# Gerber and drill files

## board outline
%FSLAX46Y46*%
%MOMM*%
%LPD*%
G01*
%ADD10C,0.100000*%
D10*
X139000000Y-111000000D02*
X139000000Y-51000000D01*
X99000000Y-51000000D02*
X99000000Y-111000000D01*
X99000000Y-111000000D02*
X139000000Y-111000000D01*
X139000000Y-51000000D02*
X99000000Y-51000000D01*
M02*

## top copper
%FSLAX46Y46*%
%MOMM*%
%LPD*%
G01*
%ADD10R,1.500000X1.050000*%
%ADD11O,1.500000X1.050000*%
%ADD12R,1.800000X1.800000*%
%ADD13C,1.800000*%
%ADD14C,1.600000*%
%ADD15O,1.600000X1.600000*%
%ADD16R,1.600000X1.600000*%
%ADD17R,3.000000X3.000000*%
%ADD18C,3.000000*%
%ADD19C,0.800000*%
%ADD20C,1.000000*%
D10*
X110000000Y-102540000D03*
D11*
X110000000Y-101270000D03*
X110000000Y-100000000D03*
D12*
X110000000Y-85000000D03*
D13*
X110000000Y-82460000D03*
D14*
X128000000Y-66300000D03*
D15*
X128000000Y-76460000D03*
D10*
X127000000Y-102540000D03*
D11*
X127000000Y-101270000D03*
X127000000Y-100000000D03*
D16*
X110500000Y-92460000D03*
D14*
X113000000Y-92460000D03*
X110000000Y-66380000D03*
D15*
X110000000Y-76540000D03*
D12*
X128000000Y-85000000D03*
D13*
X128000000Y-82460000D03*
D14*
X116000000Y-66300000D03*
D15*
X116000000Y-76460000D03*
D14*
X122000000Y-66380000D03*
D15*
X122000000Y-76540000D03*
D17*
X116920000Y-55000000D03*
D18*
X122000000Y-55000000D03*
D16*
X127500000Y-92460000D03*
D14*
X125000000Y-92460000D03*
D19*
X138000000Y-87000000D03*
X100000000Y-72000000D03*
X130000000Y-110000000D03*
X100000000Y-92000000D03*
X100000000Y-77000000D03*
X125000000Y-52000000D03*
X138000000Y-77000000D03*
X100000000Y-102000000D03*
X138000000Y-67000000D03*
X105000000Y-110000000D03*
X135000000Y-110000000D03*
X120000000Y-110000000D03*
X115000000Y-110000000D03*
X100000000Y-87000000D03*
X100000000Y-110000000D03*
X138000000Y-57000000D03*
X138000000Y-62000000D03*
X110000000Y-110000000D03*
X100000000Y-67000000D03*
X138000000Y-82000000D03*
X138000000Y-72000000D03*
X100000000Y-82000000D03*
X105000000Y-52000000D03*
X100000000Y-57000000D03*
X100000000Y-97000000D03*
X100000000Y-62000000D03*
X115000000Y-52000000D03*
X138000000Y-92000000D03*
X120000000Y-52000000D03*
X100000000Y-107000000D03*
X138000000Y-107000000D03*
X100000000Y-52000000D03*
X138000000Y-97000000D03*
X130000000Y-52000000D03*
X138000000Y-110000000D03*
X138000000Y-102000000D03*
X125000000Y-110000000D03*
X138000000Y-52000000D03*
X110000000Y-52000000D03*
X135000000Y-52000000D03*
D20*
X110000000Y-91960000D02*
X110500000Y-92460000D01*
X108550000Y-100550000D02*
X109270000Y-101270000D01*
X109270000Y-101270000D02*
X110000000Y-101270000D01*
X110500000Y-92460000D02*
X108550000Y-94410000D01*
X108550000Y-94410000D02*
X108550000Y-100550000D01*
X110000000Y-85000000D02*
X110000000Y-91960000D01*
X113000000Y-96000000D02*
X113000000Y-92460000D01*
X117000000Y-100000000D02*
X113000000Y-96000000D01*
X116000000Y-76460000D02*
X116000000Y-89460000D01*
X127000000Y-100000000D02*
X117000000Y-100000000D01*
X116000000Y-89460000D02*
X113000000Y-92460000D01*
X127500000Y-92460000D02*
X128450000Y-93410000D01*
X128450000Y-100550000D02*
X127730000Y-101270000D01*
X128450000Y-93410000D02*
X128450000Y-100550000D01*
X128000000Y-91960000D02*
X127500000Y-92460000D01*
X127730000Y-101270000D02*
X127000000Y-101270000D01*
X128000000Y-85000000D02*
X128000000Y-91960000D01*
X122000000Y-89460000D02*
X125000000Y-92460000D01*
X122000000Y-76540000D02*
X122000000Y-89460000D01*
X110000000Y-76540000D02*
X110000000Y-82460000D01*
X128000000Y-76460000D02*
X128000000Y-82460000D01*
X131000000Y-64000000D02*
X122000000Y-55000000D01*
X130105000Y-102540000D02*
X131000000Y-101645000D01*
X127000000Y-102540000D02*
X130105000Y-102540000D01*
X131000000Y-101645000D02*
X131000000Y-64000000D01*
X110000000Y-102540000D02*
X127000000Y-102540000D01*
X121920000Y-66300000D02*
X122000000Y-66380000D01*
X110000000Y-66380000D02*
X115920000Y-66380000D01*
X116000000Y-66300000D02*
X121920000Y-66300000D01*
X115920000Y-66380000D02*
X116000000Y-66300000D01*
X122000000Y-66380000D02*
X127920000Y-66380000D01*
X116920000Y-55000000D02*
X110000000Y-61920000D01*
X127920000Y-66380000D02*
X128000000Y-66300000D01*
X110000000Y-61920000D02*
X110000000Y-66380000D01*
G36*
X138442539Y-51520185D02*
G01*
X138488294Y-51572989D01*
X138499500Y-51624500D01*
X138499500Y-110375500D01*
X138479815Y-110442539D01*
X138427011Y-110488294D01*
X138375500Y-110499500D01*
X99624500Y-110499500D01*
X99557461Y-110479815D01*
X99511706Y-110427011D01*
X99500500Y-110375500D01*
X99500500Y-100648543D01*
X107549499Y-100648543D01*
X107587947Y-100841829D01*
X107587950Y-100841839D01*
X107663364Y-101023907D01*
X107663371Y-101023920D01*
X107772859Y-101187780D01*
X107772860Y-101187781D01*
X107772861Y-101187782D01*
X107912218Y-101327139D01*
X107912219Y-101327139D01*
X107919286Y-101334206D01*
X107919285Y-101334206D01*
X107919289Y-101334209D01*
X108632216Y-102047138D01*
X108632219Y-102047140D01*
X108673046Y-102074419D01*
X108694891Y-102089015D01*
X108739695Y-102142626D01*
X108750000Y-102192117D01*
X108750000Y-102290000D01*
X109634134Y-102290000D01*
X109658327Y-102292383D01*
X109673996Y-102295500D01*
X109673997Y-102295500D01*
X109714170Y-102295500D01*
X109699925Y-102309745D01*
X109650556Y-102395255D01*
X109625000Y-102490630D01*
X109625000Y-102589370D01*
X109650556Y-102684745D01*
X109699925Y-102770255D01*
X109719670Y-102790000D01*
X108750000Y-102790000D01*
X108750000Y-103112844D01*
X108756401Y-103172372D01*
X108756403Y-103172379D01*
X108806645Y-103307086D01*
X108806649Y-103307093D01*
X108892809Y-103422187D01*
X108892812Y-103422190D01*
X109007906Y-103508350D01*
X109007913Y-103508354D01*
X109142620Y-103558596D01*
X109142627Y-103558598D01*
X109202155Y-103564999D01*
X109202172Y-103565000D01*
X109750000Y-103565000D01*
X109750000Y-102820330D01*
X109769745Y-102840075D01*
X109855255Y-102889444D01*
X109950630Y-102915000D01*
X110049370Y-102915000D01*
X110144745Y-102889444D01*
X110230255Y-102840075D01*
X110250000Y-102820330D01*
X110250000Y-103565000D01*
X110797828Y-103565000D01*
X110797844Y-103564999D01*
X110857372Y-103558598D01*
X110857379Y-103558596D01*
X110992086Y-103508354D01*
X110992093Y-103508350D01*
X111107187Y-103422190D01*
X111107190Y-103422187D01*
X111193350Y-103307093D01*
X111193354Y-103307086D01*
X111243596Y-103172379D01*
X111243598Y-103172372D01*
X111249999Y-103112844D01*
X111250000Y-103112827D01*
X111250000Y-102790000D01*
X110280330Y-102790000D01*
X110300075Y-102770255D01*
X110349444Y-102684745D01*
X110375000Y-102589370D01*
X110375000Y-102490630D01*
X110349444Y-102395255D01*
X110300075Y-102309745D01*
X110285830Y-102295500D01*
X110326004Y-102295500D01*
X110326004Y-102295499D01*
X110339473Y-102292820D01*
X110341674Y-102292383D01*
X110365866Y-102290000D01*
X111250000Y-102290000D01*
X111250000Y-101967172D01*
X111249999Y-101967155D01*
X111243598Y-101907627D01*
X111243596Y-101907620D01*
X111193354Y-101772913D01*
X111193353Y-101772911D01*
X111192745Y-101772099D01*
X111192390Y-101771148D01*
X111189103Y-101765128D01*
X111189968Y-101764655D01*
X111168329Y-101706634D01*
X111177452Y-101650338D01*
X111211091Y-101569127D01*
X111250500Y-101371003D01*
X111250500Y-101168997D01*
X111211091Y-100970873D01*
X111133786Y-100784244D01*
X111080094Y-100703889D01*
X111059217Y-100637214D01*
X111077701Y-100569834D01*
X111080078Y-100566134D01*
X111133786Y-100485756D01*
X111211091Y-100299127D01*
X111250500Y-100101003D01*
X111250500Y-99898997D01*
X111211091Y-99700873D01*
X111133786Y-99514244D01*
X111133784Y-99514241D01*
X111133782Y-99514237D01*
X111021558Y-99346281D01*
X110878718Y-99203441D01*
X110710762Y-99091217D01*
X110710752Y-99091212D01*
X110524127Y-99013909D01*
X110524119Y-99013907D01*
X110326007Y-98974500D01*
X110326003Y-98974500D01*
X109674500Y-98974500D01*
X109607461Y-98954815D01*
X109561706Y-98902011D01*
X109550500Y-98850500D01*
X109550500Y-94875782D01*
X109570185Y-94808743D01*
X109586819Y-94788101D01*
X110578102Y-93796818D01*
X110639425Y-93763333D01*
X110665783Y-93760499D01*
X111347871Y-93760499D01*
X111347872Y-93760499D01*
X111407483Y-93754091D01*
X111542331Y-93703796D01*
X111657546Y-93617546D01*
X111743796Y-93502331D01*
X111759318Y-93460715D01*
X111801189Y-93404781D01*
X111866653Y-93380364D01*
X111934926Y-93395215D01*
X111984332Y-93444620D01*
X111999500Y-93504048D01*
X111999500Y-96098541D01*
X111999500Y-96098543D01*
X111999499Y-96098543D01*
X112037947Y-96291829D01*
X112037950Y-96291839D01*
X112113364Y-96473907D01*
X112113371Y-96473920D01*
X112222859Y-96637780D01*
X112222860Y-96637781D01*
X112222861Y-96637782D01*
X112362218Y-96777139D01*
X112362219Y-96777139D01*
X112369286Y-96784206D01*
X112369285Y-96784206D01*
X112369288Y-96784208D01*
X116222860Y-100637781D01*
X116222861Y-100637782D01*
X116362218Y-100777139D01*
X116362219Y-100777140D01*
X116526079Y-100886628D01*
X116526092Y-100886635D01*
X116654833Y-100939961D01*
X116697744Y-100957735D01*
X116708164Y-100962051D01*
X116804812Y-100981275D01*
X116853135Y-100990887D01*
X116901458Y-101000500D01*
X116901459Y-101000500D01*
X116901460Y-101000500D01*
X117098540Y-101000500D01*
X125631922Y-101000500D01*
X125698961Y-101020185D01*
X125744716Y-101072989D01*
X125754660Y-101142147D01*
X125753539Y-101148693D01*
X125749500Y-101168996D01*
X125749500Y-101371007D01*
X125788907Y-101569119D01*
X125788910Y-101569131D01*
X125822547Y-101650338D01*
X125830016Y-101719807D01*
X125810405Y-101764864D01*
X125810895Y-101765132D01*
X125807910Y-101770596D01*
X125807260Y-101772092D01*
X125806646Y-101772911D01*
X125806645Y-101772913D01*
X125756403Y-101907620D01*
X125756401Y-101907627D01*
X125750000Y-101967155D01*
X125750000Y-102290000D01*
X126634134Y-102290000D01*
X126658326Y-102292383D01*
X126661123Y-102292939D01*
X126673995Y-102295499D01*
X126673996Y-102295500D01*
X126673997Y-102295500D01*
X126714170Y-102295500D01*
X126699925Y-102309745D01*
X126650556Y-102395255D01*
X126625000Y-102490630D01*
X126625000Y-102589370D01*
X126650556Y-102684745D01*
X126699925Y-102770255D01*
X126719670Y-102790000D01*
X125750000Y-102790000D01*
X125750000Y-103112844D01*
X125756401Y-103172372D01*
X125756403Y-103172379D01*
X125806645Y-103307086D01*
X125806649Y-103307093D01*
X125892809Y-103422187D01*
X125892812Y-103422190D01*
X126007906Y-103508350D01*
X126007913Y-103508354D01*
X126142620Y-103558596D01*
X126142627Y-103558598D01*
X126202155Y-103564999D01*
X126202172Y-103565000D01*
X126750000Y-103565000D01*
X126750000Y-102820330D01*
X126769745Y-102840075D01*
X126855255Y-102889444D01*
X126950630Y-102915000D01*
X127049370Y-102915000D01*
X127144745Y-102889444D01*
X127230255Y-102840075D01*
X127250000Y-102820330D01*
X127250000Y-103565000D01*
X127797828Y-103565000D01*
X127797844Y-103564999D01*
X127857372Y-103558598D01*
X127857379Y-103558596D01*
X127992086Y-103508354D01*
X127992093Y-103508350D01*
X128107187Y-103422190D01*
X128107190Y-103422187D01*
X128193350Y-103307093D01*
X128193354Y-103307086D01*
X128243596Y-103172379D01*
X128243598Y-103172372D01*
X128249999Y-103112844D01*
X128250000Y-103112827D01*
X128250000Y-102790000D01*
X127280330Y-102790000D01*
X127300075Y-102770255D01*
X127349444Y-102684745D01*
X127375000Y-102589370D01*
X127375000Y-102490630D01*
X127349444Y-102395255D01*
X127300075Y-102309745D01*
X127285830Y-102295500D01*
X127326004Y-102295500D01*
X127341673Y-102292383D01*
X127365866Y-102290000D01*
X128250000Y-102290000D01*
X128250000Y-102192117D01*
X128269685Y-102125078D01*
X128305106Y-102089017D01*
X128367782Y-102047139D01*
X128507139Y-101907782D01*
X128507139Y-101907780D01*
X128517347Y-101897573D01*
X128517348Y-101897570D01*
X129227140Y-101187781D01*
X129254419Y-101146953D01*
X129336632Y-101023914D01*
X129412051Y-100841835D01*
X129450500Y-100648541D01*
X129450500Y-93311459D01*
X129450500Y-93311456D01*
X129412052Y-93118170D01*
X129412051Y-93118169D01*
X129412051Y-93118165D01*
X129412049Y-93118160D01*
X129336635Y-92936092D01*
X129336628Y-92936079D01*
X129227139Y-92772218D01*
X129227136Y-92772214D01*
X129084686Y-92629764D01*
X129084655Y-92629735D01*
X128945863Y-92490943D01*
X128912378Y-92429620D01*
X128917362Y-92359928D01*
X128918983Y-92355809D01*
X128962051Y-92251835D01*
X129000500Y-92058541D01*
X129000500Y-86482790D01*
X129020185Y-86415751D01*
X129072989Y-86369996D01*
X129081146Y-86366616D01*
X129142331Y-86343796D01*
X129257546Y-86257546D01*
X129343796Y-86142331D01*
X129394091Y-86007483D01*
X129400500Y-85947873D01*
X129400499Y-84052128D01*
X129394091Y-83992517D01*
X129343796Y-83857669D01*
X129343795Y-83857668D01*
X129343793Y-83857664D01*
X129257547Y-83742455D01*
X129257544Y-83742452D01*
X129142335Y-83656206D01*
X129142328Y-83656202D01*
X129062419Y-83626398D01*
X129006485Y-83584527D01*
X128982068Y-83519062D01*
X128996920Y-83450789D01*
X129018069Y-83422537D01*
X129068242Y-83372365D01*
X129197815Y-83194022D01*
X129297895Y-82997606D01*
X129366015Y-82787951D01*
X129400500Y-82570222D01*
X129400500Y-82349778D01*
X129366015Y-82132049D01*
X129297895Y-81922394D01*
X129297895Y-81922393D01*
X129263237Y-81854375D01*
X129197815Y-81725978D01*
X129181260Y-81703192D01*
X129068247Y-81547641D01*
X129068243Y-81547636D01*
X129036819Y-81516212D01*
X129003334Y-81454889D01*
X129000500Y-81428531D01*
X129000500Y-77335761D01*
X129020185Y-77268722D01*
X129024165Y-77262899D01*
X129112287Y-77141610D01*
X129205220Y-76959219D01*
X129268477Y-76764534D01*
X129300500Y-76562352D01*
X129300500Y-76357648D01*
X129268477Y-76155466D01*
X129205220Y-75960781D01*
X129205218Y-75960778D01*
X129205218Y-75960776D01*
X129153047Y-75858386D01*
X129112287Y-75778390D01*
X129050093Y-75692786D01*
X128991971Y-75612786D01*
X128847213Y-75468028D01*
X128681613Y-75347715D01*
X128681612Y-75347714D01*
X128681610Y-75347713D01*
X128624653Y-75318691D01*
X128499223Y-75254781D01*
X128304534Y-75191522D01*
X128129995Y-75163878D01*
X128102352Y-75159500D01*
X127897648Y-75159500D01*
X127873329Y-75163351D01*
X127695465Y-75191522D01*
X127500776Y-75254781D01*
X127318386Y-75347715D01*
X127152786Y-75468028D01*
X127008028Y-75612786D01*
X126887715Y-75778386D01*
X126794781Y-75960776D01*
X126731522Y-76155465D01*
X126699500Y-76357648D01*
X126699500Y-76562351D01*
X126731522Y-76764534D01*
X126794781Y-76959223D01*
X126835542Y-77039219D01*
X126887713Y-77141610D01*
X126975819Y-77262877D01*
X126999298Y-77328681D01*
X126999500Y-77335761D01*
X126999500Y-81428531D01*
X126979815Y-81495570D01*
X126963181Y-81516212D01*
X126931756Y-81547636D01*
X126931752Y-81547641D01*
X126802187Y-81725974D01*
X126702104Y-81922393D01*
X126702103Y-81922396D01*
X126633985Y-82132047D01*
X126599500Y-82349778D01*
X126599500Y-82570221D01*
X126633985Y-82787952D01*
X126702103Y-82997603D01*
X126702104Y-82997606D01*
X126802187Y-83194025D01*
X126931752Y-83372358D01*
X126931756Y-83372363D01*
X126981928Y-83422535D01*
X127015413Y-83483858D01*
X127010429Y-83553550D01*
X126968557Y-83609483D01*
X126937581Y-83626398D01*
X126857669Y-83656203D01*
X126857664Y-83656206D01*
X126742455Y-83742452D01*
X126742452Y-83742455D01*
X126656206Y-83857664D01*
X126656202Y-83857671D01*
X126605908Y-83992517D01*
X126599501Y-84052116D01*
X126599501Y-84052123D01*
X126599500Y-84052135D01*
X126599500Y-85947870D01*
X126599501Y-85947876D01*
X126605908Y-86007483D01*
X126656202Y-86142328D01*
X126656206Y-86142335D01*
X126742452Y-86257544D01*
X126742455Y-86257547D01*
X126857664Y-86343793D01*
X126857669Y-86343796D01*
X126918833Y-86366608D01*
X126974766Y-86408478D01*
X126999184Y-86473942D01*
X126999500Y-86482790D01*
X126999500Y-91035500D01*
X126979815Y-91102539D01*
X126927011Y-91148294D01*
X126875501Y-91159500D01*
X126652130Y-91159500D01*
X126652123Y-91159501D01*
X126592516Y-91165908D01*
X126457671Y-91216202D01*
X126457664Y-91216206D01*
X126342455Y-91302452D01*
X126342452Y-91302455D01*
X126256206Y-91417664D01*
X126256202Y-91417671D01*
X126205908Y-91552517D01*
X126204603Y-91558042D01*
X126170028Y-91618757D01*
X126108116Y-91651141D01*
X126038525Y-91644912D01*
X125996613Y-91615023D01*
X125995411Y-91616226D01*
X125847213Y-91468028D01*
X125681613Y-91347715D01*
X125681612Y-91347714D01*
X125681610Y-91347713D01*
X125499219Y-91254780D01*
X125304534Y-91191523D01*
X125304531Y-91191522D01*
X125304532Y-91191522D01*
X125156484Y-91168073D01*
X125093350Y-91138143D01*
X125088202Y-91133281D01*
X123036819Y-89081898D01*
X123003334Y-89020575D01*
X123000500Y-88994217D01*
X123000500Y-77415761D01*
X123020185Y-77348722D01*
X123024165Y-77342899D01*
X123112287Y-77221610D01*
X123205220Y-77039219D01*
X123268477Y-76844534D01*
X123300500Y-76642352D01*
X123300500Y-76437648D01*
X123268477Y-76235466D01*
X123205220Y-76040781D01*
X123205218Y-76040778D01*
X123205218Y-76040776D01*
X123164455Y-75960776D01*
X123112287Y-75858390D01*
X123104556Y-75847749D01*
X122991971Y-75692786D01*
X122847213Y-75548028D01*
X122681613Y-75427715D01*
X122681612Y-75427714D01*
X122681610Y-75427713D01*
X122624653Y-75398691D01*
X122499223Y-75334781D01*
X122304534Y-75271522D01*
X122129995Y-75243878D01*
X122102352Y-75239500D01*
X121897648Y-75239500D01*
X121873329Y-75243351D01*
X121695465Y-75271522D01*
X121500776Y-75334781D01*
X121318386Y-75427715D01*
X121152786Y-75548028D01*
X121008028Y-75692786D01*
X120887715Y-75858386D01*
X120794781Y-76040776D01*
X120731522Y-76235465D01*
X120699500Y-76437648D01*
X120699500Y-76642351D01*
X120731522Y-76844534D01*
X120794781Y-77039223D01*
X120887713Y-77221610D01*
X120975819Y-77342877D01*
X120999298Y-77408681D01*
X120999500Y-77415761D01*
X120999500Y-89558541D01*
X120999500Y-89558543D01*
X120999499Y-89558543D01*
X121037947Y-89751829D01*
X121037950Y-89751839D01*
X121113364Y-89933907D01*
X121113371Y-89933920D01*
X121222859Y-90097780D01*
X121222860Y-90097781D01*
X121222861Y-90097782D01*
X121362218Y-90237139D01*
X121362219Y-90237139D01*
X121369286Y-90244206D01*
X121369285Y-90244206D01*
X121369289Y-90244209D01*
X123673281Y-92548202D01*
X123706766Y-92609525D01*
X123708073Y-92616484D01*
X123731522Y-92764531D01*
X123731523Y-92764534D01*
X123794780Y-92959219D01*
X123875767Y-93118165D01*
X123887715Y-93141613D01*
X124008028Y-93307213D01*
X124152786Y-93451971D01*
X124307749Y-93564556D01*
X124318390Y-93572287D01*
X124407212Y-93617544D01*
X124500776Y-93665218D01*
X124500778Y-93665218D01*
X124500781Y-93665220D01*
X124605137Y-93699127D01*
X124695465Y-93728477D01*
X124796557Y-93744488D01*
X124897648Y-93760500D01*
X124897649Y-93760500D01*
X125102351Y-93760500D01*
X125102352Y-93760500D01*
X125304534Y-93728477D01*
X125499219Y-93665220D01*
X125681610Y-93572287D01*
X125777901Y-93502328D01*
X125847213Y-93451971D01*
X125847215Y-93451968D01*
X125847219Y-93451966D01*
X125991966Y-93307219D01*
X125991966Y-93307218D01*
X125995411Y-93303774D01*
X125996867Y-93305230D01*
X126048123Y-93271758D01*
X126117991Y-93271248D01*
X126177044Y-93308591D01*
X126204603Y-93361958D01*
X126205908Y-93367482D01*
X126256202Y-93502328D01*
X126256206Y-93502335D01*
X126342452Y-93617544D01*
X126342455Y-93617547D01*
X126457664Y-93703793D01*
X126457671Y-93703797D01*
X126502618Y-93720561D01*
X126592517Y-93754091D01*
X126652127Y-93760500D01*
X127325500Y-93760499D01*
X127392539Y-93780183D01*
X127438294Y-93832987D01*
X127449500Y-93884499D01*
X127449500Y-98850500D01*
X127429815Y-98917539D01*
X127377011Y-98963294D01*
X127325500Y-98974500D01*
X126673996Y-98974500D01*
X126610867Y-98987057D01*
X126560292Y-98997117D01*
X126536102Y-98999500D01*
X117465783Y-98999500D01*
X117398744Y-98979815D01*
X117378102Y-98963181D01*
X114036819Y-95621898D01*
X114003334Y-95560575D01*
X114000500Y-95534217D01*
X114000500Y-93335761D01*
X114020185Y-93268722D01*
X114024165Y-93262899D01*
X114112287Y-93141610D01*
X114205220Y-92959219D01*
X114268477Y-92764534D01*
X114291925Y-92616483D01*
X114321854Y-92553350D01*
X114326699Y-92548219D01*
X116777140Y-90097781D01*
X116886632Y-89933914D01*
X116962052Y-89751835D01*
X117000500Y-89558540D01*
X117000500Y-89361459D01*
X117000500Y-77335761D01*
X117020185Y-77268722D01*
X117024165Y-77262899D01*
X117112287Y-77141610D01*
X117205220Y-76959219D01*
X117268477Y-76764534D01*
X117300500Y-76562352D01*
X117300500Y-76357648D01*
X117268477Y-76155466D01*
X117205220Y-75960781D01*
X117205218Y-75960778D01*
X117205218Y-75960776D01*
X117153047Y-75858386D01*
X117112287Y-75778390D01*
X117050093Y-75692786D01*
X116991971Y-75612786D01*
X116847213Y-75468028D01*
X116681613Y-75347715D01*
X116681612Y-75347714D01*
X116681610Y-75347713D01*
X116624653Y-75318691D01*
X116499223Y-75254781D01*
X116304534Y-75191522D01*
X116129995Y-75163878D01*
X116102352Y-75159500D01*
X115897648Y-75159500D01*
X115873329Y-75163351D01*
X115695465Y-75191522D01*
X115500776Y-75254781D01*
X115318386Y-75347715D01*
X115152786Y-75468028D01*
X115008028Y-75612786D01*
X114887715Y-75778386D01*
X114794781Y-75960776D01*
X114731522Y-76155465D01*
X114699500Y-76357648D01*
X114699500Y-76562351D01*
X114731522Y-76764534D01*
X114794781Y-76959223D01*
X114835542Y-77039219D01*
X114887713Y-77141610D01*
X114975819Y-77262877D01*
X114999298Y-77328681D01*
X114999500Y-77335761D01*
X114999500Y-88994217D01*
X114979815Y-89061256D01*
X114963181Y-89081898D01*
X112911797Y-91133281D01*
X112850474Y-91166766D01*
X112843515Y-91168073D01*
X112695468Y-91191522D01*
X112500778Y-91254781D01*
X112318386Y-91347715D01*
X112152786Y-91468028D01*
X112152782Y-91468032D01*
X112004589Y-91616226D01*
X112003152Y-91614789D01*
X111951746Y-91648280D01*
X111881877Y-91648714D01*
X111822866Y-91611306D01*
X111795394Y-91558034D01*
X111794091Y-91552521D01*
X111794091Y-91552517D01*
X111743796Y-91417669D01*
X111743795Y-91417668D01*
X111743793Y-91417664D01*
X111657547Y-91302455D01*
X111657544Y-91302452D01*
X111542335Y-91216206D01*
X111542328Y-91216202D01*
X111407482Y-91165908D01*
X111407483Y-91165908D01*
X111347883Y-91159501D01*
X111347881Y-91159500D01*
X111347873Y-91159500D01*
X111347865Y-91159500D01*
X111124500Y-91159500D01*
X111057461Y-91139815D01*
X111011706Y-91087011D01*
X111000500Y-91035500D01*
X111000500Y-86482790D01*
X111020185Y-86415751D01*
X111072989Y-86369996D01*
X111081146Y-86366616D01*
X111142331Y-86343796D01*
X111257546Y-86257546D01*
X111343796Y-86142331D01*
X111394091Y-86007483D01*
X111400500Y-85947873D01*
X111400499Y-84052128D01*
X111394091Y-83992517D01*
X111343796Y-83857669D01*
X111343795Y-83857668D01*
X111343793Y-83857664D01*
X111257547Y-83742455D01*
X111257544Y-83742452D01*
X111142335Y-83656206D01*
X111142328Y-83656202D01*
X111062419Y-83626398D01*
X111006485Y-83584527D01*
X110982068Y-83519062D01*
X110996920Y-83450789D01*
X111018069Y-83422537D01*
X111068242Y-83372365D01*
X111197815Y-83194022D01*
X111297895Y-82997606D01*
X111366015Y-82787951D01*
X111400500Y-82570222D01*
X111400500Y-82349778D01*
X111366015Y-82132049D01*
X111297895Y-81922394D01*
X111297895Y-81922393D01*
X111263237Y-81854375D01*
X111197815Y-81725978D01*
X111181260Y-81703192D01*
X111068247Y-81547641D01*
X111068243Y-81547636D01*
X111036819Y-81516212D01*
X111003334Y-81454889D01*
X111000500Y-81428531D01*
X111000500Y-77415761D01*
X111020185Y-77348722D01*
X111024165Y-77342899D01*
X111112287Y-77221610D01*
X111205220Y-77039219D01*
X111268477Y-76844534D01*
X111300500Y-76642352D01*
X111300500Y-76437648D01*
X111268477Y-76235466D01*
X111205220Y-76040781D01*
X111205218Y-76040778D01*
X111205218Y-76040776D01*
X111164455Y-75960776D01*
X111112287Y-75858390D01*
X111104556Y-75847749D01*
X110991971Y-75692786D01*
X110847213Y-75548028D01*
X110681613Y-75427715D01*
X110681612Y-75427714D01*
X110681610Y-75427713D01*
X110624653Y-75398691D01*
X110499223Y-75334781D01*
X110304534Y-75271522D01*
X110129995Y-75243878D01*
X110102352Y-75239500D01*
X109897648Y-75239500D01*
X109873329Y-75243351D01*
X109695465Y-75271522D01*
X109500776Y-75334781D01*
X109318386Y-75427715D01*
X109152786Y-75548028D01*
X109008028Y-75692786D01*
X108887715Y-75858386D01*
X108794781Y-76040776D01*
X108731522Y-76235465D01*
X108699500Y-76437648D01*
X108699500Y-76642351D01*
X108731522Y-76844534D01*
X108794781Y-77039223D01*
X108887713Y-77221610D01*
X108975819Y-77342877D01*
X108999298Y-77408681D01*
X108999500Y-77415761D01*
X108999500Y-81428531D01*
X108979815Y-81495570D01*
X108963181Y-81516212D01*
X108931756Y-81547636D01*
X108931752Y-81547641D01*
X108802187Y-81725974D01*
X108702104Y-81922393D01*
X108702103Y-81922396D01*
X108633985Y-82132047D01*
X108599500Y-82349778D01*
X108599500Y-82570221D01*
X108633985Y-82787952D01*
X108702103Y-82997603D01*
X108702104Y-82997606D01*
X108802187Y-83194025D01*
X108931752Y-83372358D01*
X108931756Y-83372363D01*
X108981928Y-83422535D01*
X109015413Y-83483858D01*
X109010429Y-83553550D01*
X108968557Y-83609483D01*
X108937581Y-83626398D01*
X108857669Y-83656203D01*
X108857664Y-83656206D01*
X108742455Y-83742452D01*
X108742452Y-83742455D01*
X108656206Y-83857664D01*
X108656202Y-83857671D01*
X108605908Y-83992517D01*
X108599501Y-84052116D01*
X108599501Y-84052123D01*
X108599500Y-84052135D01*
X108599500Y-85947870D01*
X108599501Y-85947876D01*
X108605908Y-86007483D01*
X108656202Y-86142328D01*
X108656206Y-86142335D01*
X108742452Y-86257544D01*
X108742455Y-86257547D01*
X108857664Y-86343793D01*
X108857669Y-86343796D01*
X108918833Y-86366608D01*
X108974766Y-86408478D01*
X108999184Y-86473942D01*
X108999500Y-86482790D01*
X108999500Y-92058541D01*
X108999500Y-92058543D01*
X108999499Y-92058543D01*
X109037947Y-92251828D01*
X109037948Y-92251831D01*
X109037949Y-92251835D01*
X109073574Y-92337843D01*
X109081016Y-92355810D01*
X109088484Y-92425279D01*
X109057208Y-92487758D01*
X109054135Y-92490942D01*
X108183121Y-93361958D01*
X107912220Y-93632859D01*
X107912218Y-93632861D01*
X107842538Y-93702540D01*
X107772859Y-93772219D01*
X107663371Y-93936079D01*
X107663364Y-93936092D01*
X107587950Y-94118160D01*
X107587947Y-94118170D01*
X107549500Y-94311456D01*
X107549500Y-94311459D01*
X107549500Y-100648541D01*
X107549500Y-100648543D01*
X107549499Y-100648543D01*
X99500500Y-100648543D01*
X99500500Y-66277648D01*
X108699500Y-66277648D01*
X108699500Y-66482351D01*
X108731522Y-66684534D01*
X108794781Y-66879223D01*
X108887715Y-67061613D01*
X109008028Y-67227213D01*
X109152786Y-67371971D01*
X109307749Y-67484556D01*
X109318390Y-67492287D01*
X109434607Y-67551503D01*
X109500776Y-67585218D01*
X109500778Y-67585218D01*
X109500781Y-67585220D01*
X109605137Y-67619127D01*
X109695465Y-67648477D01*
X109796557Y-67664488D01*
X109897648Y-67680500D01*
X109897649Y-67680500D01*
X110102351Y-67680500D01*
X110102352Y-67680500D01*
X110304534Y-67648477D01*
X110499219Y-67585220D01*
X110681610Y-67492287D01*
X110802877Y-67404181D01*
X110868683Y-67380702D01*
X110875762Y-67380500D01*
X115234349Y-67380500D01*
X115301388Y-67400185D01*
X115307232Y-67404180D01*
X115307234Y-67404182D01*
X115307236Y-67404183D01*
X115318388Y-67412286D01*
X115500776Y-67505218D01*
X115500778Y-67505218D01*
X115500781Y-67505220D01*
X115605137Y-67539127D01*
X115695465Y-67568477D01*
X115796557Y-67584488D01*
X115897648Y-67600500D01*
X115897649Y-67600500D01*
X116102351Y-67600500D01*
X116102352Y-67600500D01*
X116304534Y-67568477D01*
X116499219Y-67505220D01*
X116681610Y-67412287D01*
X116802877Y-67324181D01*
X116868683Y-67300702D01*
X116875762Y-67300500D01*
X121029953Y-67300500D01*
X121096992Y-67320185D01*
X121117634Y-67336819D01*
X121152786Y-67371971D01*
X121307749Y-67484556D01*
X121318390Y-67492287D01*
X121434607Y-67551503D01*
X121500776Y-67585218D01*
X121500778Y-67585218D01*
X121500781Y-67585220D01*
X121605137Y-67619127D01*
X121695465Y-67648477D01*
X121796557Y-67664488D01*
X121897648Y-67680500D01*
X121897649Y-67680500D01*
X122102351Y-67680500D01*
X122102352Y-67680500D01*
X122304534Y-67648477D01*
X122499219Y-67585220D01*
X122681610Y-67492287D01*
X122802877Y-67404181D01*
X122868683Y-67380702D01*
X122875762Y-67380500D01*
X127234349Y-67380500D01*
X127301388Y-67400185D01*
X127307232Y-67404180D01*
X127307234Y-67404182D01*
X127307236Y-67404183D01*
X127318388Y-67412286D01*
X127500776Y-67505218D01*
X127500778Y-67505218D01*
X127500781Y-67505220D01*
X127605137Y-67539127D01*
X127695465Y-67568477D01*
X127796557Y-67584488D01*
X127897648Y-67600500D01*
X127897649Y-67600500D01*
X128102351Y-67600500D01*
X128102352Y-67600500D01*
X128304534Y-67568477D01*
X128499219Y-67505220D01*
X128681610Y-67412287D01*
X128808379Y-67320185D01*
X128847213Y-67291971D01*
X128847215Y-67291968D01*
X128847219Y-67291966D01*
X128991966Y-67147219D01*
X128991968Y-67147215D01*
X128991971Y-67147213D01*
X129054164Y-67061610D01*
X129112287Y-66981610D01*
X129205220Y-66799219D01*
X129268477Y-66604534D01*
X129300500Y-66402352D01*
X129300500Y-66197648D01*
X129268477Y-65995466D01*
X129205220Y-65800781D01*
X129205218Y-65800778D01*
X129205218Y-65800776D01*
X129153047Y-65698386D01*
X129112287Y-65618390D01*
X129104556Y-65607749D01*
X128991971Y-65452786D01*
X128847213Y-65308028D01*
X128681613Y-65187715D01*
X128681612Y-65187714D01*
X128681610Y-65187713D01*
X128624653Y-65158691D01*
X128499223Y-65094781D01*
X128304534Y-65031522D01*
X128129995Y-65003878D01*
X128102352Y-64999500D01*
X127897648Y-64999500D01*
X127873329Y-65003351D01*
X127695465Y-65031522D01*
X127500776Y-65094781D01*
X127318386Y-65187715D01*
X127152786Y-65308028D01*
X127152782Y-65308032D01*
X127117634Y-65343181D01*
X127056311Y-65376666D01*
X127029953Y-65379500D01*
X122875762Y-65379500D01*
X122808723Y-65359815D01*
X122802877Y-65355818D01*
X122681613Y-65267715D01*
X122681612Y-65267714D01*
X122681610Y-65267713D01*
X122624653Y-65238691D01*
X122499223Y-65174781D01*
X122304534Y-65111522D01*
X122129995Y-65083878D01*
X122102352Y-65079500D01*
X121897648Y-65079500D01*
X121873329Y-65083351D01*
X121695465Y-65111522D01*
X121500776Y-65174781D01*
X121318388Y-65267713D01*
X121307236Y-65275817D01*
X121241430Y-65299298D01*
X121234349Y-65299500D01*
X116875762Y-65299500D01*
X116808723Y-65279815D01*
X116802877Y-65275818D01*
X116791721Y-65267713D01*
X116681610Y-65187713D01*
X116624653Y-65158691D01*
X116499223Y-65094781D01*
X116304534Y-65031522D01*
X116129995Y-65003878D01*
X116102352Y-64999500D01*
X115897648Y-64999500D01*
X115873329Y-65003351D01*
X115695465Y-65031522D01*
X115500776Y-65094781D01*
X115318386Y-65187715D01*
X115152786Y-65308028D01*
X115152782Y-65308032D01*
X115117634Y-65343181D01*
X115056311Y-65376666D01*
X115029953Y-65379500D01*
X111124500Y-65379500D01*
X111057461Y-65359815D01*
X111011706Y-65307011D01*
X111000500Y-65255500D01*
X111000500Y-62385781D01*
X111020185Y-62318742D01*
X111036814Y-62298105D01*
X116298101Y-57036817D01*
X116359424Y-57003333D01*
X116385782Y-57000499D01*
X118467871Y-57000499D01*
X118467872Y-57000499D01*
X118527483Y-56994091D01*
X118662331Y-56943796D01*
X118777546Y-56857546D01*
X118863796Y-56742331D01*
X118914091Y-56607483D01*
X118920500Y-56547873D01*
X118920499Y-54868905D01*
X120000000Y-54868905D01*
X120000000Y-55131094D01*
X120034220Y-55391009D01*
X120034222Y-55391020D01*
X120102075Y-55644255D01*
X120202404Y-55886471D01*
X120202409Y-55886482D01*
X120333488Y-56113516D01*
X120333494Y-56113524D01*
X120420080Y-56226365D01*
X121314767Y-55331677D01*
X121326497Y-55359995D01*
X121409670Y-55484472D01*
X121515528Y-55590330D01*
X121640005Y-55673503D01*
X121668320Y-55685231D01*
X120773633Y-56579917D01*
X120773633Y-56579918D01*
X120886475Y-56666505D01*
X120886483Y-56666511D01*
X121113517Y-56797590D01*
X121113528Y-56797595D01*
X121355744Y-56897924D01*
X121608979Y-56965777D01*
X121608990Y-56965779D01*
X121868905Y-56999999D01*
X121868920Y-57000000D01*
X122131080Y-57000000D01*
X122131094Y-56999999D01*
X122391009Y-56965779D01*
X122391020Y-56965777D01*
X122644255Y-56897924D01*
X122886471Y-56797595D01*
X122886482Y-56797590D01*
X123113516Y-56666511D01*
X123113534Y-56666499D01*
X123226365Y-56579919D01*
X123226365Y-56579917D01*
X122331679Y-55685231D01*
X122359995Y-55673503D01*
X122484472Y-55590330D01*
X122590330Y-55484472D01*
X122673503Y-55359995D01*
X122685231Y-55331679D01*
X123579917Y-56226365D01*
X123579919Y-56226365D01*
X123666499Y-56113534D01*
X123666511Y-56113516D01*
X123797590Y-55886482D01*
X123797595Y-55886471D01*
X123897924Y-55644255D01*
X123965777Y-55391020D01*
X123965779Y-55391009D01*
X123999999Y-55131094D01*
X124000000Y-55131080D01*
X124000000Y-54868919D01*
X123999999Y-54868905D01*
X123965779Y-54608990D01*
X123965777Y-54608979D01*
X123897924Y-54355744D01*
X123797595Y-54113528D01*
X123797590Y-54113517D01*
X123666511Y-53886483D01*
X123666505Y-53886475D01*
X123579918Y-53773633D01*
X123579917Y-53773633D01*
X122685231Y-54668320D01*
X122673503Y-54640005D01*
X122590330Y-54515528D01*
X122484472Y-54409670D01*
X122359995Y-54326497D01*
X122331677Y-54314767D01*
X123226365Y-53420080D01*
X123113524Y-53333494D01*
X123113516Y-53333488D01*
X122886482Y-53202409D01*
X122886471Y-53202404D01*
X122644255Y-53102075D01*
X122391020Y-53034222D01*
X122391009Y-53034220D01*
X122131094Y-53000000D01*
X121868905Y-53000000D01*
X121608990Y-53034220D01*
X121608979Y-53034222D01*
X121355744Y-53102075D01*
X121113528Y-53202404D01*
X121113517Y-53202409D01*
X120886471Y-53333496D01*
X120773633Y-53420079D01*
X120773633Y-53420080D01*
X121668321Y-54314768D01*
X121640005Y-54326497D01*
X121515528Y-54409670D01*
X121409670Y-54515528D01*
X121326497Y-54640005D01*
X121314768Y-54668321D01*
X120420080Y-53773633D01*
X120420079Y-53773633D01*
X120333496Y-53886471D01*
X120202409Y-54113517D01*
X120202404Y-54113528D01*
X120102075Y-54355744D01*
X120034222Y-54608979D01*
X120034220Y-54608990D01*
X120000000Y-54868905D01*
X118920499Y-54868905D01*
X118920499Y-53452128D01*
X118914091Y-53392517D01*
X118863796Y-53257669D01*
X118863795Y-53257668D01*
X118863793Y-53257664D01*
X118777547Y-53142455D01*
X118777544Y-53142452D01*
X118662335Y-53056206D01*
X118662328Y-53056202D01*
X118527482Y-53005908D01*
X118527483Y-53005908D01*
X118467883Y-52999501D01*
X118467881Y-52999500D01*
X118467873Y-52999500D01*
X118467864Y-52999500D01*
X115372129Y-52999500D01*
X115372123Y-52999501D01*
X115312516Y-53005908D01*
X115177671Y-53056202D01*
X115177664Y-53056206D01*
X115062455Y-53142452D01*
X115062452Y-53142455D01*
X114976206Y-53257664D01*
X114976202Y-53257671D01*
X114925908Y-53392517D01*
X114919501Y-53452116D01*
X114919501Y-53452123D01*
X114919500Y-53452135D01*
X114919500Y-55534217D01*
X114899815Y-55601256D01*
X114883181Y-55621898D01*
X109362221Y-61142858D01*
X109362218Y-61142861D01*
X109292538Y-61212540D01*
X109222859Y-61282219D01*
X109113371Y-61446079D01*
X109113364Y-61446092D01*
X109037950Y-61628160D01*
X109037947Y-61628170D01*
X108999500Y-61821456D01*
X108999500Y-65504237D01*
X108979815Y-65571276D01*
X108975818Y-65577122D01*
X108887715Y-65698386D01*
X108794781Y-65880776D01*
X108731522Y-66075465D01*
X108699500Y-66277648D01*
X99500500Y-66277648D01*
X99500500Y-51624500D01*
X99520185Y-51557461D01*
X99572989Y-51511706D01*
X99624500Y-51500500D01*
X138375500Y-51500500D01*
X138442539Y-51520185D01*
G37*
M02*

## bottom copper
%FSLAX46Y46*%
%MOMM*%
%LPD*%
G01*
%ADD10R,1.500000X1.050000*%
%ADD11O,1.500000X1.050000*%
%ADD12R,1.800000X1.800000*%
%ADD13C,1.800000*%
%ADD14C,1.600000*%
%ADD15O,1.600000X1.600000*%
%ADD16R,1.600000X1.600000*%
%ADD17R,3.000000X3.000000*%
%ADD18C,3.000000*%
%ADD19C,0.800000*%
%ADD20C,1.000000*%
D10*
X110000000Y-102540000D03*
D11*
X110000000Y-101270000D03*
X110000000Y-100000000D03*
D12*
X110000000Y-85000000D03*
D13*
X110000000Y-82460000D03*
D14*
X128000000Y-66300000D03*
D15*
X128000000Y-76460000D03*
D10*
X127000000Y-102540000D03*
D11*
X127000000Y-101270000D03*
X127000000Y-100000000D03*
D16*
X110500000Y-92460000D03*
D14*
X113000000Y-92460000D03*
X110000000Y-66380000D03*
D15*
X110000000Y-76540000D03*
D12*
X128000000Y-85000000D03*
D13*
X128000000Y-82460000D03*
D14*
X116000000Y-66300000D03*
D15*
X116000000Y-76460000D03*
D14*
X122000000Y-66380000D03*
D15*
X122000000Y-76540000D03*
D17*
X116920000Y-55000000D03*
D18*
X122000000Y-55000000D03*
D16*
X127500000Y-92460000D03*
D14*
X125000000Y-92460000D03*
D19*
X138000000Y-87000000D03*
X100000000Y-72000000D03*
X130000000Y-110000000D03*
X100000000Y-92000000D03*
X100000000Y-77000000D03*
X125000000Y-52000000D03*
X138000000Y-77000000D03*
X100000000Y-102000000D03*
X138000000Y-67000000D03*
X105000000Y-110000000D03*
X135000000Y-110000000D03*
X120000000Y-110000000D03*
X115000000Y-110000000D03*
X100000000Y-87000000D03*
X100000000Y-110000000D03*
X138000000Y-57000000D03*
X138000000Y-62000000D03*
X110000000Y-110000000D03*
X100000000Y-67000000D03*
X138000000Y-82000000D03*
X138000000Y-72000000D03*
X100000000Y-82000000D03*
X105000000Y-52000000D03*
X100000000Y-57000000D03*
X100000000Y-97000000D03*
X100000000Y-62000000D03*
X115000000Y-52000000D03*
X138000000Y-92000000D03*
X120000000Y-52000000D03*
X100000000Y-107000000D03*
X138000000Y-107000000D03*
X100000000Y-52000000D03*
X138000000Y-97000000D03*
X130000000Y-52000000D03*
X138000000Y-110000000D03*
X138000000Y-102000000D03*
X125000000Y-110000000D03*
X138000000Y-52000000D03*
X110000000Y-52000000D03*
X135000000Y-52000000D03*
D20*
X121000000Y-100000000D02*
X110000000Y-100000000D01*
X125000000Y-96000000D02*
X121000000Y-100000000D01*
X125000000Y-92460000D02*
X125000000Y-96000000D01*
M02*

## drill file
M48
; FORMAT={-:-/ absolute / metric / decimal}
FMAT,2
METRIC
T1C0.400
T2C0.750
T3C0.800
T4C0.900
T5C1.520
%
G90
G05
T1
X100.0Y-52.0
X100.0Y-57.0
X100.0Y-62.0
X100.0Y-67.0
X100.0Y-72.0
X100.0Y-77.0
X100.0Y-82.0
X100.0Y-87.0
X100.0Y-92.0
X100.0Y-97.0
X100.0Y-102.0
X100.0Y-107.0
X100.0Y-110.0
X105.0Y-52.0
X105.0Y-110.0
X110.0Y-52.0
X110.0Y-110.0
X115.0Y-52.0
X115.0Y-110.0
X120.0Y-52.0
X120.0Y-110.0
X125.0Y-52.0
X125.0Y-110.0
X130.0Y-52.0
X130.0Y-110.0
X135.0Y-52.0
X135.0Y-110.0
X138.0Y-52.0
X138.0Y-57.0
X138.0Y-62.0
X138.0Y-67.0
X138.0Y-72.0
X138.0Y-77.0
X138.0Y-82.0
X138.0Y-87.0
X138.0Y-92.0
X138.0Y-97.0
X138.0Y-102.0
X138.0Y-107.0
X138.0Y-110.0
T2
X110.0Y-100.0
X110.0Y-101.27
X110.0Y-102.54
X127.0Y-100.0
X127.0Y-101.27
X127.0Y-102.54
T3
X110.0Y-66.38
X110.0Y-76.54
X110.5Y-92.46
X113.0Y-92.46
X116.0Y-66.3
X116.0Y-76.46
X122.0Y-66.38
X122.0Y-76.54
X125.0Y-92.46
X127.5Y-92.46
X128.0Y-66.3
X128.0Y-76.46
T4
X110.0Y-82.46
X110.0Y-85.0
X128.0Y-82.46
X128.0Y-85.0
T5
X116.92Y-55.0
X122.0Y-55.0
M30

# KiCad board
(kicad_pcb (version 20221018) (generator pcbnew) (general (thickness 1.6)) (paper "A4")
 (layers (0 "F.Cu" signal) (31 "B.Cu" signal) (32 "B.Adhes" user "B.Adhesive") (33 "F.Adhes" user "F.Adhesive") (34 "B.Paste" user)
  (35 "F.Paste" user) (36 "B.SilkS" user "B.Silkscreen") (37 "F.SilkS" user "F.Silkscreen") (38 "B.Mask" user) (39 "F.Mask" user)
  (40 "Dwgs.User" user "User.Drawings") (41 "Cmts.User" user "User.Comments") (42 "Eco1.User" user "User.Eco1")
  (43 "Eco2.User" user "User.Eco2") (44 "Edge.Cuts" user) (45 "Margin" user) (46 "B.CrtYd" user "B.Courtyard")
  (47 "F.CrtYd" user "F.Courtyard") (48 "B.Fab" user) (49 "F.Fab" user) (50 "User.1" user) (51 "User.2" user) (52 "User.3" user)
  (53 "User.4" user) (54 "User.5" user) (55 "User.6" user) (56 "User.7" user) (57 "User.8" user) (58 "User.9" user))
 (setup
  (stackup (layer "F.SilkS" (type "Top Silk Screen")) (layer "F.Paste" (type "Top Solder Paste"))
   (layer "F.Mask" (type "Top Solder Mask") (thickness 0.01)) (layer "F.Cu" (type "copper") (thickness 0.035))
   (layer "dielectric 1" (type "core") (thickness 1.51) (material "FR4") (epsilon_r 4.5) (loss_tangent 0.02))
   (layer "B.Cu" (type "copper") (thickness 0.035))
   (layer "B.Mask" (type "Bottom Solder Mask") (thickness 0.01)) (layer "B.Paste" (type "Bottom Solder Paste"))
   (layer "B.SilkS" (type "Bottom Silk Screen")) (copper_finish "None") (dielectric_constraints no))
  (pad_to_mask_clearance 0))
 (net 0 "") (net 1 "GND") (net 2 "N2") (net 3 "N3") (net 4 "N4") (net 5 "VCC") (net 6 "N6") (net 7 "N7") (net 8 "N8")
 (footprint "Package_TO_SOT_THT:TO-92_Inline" (layer "F.Cu") (at 110 102.54 90)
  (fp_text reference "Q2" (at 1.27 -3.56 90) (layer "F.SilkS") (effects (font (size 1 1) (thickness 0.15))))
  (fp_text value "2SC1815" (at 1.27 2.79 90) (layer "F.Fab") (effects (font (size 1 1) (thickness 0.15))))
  (pad "1" thru_hole rect (at 0 0 90) (size 1.05 1.5) (drill 0.75) (layers "*.Cu" "*.Mask") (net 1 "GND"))
  (pad "2" thru_hole oval (at 1.27 0 90) (size 1.05 1.5) (drill 0.75) (layers "*.Cu" "*.Mask") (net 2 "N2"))
  (pad "3" thru_hole oval (at 2.54 0 90) (size 1.05 1.5) (drill 0.75) (layers "*.Cu" "*.Mask") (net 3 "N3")))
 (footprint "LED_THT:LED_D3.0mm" (layer "F.Cu") (at 110 85 90)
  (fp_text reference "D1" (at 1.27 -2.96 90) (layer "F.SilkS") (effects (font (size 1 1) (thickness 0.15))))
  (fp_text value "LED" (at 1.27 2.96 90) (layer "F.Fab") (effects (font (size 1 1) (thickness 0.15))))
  (pad "1" thru_hole rect (at 0 0 90) (size 1.8 1.8) (drill 0.9) (layers "*.Cu" "*.Mask") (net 2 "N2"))
  (pad "2" thru_hole circle (at 2.54 0 90) (size 1.8 1.8) (drill 0.9) (layers "*.Cu" "*.Mask") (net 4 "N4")))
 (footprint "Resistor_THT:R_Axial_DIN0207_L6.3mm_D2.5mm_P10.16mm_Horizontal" (layer "F.Cu") (at 128 66.3 -90)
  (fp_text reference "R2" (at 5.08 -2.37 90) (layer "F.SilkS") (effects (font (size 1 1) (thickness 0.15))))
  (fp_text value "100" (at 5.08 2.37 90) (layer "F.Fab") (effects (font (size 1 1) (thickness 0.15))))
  (pad "1" thru_hole circle (at 0 0 270) (size 1.6 1.6) (drill 0.8) (layers "*.Cu" "*.Mask") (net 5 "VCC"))
  (pad "2" thru_hole oval (at 10.16 0 270) (size 1.6 1.6) (drill 0.8) (layers "*.Cu" "*.Mask") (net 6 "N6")))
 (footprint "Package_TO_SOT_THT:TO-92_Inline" (layer "F.Cu") (at 127 102.54 90)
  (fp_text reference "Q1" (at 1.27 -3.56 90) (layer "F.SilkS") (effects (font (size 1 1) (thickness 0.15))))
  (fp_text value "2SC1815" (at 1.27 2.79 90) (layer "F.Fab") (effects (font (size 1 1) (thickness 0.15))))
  (pad "1" thru_hole rect (at 0 0 90) (size 1.05 1.5) (drill 0.75) (layers "*.Cu" "*.Mask") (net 1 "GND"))
  (pad "2" thru_hole oval (at 1.27 0 90) (size 1.05 1.5) (drill 0.75) (layers "*.Cu" "*.Mask") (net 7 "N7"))
  (pad "3" thru_hole oval (at 2.54 0 90) (size 1.05 1.5) (drill 0.75) (layers "*.Cu" "*.Mask") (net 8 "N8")))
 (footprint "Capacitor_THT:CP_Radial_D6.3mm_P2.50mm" (layer "F.Cu") (at 110.5 92.46)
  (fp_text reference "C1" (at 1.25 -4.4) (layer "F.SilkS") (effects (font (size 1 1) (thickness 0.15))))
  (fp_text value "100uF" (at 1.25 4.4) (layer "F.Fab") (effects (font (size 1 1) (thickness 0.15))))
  (pad "1" thru_hole rect (at 0 0) (size 1.6 1.6) (drill 0.8) (layers "*.Cu" "*.Mask") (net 2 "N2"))
  (pad "2" thru_hole circle (at 2.5 0) (size 1.6 1.6) (drill 0.8) (layers "*.Cu" "*.Mask") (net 8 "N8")))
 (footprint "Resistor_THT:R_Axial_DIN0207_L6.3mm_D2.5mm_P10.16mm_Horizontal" (layer "F.Cu") (at 110 66.38 -90)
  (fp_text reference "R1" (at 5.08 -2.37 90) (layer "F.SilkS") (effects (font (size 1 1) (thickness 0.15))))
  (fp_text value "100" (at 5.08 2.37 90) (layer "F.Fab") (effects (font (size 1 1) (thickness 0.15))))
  (pad "1" thru_hole circle (at 0 0 270) (size 1.6 1.6) (drill 0.8) (layers "*.Cu" "*.Mask") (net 5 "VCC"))
  (pad "2" thru_hole oval (at 10.16 0 270) (size 1.6 1.6) (drill 0.8) (layers "*.Cu" "*.Mask") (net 4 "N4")))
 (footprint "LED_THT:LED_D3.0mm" (layer "F.Cu") (at 128 85 90)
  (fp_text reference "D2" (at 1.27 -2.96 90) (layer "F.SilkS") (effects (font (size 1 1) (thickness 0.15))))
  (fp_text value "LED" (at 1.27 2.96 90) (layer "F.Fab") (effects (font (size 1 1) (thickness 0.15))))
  (pad "1" thru_hole rect (at 0 0 90) (size 1.8 1.8) (drill 0.9) (layers "*.Cu" "*.Mask") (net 7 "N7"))
  (pad "2" thru_hole circle (at 2.54 0 90) (size 1.8 1.8) (drill 0.9) (layers "*.Cu" "*.Mask") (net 6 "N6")))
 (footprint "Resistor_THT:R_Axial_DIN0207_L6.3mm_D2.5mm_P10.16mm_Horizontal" (layer "F.Cu") (at 116 66.3 -90)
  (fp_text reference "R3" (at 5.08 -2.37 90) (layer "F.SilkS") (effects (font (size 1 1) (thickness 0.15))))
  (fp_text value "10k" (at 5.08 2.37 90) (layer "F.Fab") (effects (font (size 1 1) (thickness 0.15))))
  (pad "1" thru_hole circle (at 0 0 270) (size 1.6 1.6) (drill 0.8) (layers "*.Cu" "*.Mask") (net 5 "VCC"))
  (pad "2" thru_hole oval (at 10.16 0 270) (size 1.6 1.6) (drill 0.8) (layers "*.Cu" "*.Mask") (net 8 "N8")))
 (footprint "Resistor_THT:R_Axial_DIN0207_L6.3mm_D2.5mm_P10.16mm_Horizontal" (layer "F.Cu") (at 122 66.38 -90)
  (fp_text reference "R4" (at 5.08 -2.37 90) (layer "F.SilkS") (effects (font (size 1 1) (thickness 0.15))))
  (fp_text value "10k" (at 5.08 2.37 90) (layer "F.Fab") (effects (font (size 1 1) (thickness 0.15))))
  (pad "1" thru_hole circle (at 0 0 270) (size 1.6 1.6) (drill 0.8) (layers "*.Cu" "*.Mask") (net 5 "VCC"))
  (pad "2" thru_hole oval (at 10.16 0 270) (size 1.6 1.6) (drill 0.8) (layers "*.Cu" "*.Mask") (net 3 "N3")))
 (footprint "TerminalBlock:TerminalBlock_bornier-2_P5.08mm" (layer "F.Cu") (at 116.92 55)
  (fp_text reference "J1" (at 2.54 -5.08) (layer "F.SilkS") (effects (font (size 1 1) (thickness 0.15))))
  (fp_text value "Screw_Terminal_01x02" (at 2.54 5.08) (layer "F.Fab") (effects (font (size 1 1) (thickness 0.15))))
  (pad "1" thru_hole rect (at 0 0) (size 3 3) (drill 1.52) (layers "*.Cu" "*.Mask") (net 5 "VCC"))
  (pad "2" thru_hole circle (at 5.08 0) (size 3 3) (drill 1.52) (layers "*.Cu" "*.Mask") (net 1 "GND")))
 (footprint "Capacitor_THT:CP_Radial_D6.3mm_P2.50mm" (layer "F.Cu") (at 127.5 92.46 180)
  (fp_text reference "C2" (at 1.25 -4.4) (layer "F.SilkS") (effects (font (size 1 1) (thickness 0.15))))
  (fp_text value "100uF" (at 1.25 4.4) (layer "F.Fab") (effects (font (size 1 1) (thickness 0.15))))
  (pad "1" thru_hole rect (at 0 0 180) (size 1.6 1.6) (drill 0.8) (layers "*.Cu" "*.Mask") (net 7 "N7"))
  (pad "2" thru_hole circle (at 2.5 0 180) (size 1.6 1.6) (drill 0.8) (layers "*.Cu" "*.Mask") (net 3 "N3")))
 (gr_line (start 139 111) (end 139 51) (stroke (width 0.1) (type default)) (layer "Edge.Cuts"))
 (gr_line (start 99 51) (end 99 111) (stroke (width 0.1) (type default)) (layer "Edge.Cuts"))
 (gr_line (start 99 111) (end 139 111) (stroke (width 0.1) (type default)) (layer "Edge.Cuts"))
 (gr_line (start 139 51) (end 99 51) (stroke (width 0.1) (type default)) (layer "Edge.Cuts"))
 (segment (start 110 91.96) (end 110.5 92.46) (width 1) (layer "F.Cu") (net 2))
 (segment (start 108.55 100.55) (end 109.27 101.27) (width 1) (layer "F.Cu") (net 2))
 (segment (start 109.27 101.27) (end 110 101.27) (width 1) (layer "F.Cu") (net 2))
 (segment (start 110.5 92.46) (end 108.55 94.41) (width 1) (layer "F.Cu") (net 2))
 (segment (start 108.55 94.41) (end 108.55 100.55) (width 1) (layer "F.Cu") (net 2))
 (segment (start 110 85) (end 110 91.96) (width 1) (layer "F.Cu") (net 2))
 (segment (start 113 96) (end 113 92.46) (width 1) (layer "F.Cu") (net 8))
 (segment (start 117 100) (end 113 96) (width 1) (layer "F.Cu") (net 8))
 (segment (start 116 76.46) (end 116 89.46) (width 1) (layer "F.Cu") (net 8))
 (segment (start 127 100) (end 117 100) (width 1) (layer "F.Cu") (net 8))
 (segment (start 116 89.46) (end 113 92.46) (width 1) (layer "F.Cu") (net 8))
 (segment (start 127.5 92.46) (end 128.45 93.41) (width 1) (layer "F.Cu") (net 7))
 (segment (start 128.45 100.55) (end 127.73 101.27) (width 1) (layer "F.Cu") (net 7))
 (segment (start 128.45 93.41) (end 128.45 100.55) (width 1) (layer "F.Cu") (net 7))
 (segment (start 128 91.96) (end 127.5 92.46) (width 1) (layer "F.Cu") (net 7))
 (segment (start 127.73 101.27) (end 127 101.27) (width 1) (layer "F.Cu") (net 7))
 (segment (start 128 85) (end 128 91.96) (width 1) (layer "F.Cu") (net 7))
 (segment (start 122 89.46) (end 125 92.46) (width 1) (layer "F.Cu") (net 3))
 (segment (start 122 76.54) (end 122 89.46) (width 1) (layer "F.Cu") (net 3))
 (segment (start 121 100) (end 110 100) (width 1) (layer "B.Cu") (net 3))
 (segment (start 125 96) (end 121 100) (width 1) (layer "B.Cu") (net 3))
 (segment (start 125 92.46) (end 125 96) (width 1) (layer "B.Cu") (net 3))
 (segment (start 110 76.54) (end 110 82.46) (width 1) (layer "F.Cu") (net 4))
 (segment (start 128 76.46) (end 128 82.46) (width 1) (layer "F.Cu") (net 6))
 (segment (start 131 64) (end 122 55) (width 1) (layer "F.Cu") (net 1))
 (segment (start 130.105 102.54) (end 131 101.645) (width 1) (layer "F.Cu") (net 1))
 (segment (start 127 102.54) (end 130.105 102.54) (width 1) (layer "F.Cu") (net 1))
 (segment (start 131 101.645) (end 131 64) (width 1) (layer "F.Cu") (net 1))
 (segment (start 110 102.54) (end 127 102.54) (width 1) (layer "F.Cu") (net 1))
 (via (at 138 87) (size 0.8) (drill 0.4) (layers "F.Cu" "B.Cu") (free) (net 1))
 (via (at 100 72) (size 0.8) (drill 0.4) (layers "F.Cu" "B.Cu") (free) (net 1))
 (via (at 130 110) (size 0.8) (drill 0.4) (layers "F.Cu" "B.Cu") (free) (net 1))
 (via (at 100 92) (size 0.8) (drill 0.4) (layers "F.Cu" "B.Cu") (free) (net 1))
 (via (at 100 77) (size 0.8) (drill 0.4) (layers "F.Cu" "B.Cu") (free) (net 1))
 (via (at 125 52) (size 0.8) (drill 0.4) (layers "F.Cu" "B.Cu") (free) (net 1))
 (via (at 138 77) (size 0.8) (drill 0.4) (layers "F.Cu" "B.Cu") (free) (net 1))
 (via (at 100 102) (size 0.8) (drill 0.4) (layers "F.Cu" "B.Cu") (free) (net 1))
 (via (at 138 67) (size 0.8) (drill 0.4) (layers "F.Cu" "B.Cu") (free) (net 1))
 (via (at 105 110) (size 0.8) (drill 0.4) (layers "F.Cu" "B.Cu") (free) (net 1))
 (via (at 135 110) (size 0.8) (drill 0.4) (layers "F.Cu" "B.Cu") (free) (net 1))
 (via (at 120 110) (size 0.8) (drill 0.4) (layers "F.Cu" "B.Cu") (free) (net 1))
 (via (at 115 110) (size 0.8) (drill 0.4) (layers "F.Cu" "B.Cu") (free) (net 1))
 (via (at 100 87) (size 0.8) (drill 0.4) (layers "F.Cu" "B.Cu") (free) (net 1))
 (via (at 100 110) (size 0.8) (drill 0.4) (layers "F.Cu" "B.Cu") (free) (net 1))
 (via (at 138 57) (size 0.8) (drill 0.4) (layers "F.Cu" "B.Cu") (free) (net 1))
 (via (at 138 62) (size 0.8) (drill 0.4) (layers "F.Cu" "B.Cu") (free) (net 1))
 (via (at 110 110) (size 0.8) (drill 0.4) (layers "F.Cu" "B.Cu") (free) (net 1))
 (via (at 100 67) (size 0.8) (drill 0.4) (layers "F.Cu" "B.Cu") (free) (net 1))
 (via (at 138 82) (size 0.8) (drill 0.4) (layers "F.Cu" "B.Cu") (free) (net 1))
 (via (at 138 72) (size 0.8) (drill 0.4) (layers "F.Cu" "B.Cu") (free) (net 1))
 (via (at 100 82) (size 0.8) (drill 0.4) (layers "F.Cu" "B.Cu") (free) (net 1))
 (via (at 105 52) (size 0.8) (drill 0.4) (layers "F.Cu" "B.Cu") (free) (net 1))
 (via (at 100 57) (size 0.8) (drill 0.4) (layers "F.Cu" "B.Cu") (free) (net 1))
 (via (at 100 97) (size 0.8) (drill 0.4) (layers "F.Cu" "B.Cu") (free) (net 1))
 (via (at 100 62) (size 0.8) (drill 0.4) (layers "F.Cu" "B.Cu") (free) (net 1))
 (via (at 115 52) (size 0.8) (drill 0.4) (layers "F.Cu" "B.Cu") (free) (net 1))
 (via (at 138 92) (size 0.8) (drill 0.4) (layers "F.Cu" "B.Cu") (free) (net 1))
 (via (at 120 52) (size 0.8) (drill 0.4) (layers "F.Cu" "B.Cu") (free) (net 1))
 (via (at 100 107) (size 0.8) (drill 0.4) (layers "F.Cu" "B.Cu") (free) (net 1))
 (via (at 138 107) (size 0.8) (drill 0.4) (layers "F.Cu" "B.Cu") (free) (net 1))
 (via (at 100 52) (size 0.8) (drill 0.4) (layers "F.Cu" "B.Cu") (free) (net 1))
 (via (at 138 97) (size 0.8) (drill 0.4) (layers "F.Cu" "B.Cu") (free) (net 1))
 (via (at 130 52) (size 0.8) (drill 0.4) (layers "F.Cu" "B.Cu") (free) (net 1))
 (via (at 138 110) (size 0.8) (drill 0.4) (layers "F.Cu" "B.Cu") (free) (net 1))
 (via (at 138 102) (size 0.8) (drill 0.4) (layers "F.Cu" "B.Cu") (free) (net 1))
 (via (at 125 110) (size 0.8) (drill 0.4) (layers "F.Cu" "B.Cu") (free) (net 1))
 (via (at 138 52) (size 0.8) (drill 0.4) (layers "F.Cu" "B.Cu") (free) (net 1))
 (via (at 110 52) (size 0.8) (drill 0.4) (layers "F.Cu" "B.Cu") (free) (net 1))
 (via (at 135 52) (size 0.8) (drill 0.4) (layers "F.Cu" "B.Cu") (free) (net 1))
 (segment (start 121.92 66.3) (end 122 66.38) (width 1) (layer "F.Cu") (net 5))
 (segment (start 110 66.38) (end 115.92 66.38) (width 1) (layer "F.Cu") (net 5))
 (segment (start 116 66.3) (end 121.92 66.3) (width 1) (layer "F.Cu") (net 5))
 (segment (start 115.92 66.38) (end 116 66.3) (width 1) (layer "F.Cu") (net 5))
 (segment (start 122 66.38) (end 127.92 66.38) (width 1) (layer "F.Cu") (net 5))
 (segment (start 116.92 55) (end 110 61.92) (width 1) (layer "F.Cu") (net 5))
 (segment (start 127.92 66.38) (end 128 66.3) (width 1) (layer "F.Cu") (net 5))
 (segment (start 110 61.92) (end 110 66.38) (width 1) (layer "F.Cu") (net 5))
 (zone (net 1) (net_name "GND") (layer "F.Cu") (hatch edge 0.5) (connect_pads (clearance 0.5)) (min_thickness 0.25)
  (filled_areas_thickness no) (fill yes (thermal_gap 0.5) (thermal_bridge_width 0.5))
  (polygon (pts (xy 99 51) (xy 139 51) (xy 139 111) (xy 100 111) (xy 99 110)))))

